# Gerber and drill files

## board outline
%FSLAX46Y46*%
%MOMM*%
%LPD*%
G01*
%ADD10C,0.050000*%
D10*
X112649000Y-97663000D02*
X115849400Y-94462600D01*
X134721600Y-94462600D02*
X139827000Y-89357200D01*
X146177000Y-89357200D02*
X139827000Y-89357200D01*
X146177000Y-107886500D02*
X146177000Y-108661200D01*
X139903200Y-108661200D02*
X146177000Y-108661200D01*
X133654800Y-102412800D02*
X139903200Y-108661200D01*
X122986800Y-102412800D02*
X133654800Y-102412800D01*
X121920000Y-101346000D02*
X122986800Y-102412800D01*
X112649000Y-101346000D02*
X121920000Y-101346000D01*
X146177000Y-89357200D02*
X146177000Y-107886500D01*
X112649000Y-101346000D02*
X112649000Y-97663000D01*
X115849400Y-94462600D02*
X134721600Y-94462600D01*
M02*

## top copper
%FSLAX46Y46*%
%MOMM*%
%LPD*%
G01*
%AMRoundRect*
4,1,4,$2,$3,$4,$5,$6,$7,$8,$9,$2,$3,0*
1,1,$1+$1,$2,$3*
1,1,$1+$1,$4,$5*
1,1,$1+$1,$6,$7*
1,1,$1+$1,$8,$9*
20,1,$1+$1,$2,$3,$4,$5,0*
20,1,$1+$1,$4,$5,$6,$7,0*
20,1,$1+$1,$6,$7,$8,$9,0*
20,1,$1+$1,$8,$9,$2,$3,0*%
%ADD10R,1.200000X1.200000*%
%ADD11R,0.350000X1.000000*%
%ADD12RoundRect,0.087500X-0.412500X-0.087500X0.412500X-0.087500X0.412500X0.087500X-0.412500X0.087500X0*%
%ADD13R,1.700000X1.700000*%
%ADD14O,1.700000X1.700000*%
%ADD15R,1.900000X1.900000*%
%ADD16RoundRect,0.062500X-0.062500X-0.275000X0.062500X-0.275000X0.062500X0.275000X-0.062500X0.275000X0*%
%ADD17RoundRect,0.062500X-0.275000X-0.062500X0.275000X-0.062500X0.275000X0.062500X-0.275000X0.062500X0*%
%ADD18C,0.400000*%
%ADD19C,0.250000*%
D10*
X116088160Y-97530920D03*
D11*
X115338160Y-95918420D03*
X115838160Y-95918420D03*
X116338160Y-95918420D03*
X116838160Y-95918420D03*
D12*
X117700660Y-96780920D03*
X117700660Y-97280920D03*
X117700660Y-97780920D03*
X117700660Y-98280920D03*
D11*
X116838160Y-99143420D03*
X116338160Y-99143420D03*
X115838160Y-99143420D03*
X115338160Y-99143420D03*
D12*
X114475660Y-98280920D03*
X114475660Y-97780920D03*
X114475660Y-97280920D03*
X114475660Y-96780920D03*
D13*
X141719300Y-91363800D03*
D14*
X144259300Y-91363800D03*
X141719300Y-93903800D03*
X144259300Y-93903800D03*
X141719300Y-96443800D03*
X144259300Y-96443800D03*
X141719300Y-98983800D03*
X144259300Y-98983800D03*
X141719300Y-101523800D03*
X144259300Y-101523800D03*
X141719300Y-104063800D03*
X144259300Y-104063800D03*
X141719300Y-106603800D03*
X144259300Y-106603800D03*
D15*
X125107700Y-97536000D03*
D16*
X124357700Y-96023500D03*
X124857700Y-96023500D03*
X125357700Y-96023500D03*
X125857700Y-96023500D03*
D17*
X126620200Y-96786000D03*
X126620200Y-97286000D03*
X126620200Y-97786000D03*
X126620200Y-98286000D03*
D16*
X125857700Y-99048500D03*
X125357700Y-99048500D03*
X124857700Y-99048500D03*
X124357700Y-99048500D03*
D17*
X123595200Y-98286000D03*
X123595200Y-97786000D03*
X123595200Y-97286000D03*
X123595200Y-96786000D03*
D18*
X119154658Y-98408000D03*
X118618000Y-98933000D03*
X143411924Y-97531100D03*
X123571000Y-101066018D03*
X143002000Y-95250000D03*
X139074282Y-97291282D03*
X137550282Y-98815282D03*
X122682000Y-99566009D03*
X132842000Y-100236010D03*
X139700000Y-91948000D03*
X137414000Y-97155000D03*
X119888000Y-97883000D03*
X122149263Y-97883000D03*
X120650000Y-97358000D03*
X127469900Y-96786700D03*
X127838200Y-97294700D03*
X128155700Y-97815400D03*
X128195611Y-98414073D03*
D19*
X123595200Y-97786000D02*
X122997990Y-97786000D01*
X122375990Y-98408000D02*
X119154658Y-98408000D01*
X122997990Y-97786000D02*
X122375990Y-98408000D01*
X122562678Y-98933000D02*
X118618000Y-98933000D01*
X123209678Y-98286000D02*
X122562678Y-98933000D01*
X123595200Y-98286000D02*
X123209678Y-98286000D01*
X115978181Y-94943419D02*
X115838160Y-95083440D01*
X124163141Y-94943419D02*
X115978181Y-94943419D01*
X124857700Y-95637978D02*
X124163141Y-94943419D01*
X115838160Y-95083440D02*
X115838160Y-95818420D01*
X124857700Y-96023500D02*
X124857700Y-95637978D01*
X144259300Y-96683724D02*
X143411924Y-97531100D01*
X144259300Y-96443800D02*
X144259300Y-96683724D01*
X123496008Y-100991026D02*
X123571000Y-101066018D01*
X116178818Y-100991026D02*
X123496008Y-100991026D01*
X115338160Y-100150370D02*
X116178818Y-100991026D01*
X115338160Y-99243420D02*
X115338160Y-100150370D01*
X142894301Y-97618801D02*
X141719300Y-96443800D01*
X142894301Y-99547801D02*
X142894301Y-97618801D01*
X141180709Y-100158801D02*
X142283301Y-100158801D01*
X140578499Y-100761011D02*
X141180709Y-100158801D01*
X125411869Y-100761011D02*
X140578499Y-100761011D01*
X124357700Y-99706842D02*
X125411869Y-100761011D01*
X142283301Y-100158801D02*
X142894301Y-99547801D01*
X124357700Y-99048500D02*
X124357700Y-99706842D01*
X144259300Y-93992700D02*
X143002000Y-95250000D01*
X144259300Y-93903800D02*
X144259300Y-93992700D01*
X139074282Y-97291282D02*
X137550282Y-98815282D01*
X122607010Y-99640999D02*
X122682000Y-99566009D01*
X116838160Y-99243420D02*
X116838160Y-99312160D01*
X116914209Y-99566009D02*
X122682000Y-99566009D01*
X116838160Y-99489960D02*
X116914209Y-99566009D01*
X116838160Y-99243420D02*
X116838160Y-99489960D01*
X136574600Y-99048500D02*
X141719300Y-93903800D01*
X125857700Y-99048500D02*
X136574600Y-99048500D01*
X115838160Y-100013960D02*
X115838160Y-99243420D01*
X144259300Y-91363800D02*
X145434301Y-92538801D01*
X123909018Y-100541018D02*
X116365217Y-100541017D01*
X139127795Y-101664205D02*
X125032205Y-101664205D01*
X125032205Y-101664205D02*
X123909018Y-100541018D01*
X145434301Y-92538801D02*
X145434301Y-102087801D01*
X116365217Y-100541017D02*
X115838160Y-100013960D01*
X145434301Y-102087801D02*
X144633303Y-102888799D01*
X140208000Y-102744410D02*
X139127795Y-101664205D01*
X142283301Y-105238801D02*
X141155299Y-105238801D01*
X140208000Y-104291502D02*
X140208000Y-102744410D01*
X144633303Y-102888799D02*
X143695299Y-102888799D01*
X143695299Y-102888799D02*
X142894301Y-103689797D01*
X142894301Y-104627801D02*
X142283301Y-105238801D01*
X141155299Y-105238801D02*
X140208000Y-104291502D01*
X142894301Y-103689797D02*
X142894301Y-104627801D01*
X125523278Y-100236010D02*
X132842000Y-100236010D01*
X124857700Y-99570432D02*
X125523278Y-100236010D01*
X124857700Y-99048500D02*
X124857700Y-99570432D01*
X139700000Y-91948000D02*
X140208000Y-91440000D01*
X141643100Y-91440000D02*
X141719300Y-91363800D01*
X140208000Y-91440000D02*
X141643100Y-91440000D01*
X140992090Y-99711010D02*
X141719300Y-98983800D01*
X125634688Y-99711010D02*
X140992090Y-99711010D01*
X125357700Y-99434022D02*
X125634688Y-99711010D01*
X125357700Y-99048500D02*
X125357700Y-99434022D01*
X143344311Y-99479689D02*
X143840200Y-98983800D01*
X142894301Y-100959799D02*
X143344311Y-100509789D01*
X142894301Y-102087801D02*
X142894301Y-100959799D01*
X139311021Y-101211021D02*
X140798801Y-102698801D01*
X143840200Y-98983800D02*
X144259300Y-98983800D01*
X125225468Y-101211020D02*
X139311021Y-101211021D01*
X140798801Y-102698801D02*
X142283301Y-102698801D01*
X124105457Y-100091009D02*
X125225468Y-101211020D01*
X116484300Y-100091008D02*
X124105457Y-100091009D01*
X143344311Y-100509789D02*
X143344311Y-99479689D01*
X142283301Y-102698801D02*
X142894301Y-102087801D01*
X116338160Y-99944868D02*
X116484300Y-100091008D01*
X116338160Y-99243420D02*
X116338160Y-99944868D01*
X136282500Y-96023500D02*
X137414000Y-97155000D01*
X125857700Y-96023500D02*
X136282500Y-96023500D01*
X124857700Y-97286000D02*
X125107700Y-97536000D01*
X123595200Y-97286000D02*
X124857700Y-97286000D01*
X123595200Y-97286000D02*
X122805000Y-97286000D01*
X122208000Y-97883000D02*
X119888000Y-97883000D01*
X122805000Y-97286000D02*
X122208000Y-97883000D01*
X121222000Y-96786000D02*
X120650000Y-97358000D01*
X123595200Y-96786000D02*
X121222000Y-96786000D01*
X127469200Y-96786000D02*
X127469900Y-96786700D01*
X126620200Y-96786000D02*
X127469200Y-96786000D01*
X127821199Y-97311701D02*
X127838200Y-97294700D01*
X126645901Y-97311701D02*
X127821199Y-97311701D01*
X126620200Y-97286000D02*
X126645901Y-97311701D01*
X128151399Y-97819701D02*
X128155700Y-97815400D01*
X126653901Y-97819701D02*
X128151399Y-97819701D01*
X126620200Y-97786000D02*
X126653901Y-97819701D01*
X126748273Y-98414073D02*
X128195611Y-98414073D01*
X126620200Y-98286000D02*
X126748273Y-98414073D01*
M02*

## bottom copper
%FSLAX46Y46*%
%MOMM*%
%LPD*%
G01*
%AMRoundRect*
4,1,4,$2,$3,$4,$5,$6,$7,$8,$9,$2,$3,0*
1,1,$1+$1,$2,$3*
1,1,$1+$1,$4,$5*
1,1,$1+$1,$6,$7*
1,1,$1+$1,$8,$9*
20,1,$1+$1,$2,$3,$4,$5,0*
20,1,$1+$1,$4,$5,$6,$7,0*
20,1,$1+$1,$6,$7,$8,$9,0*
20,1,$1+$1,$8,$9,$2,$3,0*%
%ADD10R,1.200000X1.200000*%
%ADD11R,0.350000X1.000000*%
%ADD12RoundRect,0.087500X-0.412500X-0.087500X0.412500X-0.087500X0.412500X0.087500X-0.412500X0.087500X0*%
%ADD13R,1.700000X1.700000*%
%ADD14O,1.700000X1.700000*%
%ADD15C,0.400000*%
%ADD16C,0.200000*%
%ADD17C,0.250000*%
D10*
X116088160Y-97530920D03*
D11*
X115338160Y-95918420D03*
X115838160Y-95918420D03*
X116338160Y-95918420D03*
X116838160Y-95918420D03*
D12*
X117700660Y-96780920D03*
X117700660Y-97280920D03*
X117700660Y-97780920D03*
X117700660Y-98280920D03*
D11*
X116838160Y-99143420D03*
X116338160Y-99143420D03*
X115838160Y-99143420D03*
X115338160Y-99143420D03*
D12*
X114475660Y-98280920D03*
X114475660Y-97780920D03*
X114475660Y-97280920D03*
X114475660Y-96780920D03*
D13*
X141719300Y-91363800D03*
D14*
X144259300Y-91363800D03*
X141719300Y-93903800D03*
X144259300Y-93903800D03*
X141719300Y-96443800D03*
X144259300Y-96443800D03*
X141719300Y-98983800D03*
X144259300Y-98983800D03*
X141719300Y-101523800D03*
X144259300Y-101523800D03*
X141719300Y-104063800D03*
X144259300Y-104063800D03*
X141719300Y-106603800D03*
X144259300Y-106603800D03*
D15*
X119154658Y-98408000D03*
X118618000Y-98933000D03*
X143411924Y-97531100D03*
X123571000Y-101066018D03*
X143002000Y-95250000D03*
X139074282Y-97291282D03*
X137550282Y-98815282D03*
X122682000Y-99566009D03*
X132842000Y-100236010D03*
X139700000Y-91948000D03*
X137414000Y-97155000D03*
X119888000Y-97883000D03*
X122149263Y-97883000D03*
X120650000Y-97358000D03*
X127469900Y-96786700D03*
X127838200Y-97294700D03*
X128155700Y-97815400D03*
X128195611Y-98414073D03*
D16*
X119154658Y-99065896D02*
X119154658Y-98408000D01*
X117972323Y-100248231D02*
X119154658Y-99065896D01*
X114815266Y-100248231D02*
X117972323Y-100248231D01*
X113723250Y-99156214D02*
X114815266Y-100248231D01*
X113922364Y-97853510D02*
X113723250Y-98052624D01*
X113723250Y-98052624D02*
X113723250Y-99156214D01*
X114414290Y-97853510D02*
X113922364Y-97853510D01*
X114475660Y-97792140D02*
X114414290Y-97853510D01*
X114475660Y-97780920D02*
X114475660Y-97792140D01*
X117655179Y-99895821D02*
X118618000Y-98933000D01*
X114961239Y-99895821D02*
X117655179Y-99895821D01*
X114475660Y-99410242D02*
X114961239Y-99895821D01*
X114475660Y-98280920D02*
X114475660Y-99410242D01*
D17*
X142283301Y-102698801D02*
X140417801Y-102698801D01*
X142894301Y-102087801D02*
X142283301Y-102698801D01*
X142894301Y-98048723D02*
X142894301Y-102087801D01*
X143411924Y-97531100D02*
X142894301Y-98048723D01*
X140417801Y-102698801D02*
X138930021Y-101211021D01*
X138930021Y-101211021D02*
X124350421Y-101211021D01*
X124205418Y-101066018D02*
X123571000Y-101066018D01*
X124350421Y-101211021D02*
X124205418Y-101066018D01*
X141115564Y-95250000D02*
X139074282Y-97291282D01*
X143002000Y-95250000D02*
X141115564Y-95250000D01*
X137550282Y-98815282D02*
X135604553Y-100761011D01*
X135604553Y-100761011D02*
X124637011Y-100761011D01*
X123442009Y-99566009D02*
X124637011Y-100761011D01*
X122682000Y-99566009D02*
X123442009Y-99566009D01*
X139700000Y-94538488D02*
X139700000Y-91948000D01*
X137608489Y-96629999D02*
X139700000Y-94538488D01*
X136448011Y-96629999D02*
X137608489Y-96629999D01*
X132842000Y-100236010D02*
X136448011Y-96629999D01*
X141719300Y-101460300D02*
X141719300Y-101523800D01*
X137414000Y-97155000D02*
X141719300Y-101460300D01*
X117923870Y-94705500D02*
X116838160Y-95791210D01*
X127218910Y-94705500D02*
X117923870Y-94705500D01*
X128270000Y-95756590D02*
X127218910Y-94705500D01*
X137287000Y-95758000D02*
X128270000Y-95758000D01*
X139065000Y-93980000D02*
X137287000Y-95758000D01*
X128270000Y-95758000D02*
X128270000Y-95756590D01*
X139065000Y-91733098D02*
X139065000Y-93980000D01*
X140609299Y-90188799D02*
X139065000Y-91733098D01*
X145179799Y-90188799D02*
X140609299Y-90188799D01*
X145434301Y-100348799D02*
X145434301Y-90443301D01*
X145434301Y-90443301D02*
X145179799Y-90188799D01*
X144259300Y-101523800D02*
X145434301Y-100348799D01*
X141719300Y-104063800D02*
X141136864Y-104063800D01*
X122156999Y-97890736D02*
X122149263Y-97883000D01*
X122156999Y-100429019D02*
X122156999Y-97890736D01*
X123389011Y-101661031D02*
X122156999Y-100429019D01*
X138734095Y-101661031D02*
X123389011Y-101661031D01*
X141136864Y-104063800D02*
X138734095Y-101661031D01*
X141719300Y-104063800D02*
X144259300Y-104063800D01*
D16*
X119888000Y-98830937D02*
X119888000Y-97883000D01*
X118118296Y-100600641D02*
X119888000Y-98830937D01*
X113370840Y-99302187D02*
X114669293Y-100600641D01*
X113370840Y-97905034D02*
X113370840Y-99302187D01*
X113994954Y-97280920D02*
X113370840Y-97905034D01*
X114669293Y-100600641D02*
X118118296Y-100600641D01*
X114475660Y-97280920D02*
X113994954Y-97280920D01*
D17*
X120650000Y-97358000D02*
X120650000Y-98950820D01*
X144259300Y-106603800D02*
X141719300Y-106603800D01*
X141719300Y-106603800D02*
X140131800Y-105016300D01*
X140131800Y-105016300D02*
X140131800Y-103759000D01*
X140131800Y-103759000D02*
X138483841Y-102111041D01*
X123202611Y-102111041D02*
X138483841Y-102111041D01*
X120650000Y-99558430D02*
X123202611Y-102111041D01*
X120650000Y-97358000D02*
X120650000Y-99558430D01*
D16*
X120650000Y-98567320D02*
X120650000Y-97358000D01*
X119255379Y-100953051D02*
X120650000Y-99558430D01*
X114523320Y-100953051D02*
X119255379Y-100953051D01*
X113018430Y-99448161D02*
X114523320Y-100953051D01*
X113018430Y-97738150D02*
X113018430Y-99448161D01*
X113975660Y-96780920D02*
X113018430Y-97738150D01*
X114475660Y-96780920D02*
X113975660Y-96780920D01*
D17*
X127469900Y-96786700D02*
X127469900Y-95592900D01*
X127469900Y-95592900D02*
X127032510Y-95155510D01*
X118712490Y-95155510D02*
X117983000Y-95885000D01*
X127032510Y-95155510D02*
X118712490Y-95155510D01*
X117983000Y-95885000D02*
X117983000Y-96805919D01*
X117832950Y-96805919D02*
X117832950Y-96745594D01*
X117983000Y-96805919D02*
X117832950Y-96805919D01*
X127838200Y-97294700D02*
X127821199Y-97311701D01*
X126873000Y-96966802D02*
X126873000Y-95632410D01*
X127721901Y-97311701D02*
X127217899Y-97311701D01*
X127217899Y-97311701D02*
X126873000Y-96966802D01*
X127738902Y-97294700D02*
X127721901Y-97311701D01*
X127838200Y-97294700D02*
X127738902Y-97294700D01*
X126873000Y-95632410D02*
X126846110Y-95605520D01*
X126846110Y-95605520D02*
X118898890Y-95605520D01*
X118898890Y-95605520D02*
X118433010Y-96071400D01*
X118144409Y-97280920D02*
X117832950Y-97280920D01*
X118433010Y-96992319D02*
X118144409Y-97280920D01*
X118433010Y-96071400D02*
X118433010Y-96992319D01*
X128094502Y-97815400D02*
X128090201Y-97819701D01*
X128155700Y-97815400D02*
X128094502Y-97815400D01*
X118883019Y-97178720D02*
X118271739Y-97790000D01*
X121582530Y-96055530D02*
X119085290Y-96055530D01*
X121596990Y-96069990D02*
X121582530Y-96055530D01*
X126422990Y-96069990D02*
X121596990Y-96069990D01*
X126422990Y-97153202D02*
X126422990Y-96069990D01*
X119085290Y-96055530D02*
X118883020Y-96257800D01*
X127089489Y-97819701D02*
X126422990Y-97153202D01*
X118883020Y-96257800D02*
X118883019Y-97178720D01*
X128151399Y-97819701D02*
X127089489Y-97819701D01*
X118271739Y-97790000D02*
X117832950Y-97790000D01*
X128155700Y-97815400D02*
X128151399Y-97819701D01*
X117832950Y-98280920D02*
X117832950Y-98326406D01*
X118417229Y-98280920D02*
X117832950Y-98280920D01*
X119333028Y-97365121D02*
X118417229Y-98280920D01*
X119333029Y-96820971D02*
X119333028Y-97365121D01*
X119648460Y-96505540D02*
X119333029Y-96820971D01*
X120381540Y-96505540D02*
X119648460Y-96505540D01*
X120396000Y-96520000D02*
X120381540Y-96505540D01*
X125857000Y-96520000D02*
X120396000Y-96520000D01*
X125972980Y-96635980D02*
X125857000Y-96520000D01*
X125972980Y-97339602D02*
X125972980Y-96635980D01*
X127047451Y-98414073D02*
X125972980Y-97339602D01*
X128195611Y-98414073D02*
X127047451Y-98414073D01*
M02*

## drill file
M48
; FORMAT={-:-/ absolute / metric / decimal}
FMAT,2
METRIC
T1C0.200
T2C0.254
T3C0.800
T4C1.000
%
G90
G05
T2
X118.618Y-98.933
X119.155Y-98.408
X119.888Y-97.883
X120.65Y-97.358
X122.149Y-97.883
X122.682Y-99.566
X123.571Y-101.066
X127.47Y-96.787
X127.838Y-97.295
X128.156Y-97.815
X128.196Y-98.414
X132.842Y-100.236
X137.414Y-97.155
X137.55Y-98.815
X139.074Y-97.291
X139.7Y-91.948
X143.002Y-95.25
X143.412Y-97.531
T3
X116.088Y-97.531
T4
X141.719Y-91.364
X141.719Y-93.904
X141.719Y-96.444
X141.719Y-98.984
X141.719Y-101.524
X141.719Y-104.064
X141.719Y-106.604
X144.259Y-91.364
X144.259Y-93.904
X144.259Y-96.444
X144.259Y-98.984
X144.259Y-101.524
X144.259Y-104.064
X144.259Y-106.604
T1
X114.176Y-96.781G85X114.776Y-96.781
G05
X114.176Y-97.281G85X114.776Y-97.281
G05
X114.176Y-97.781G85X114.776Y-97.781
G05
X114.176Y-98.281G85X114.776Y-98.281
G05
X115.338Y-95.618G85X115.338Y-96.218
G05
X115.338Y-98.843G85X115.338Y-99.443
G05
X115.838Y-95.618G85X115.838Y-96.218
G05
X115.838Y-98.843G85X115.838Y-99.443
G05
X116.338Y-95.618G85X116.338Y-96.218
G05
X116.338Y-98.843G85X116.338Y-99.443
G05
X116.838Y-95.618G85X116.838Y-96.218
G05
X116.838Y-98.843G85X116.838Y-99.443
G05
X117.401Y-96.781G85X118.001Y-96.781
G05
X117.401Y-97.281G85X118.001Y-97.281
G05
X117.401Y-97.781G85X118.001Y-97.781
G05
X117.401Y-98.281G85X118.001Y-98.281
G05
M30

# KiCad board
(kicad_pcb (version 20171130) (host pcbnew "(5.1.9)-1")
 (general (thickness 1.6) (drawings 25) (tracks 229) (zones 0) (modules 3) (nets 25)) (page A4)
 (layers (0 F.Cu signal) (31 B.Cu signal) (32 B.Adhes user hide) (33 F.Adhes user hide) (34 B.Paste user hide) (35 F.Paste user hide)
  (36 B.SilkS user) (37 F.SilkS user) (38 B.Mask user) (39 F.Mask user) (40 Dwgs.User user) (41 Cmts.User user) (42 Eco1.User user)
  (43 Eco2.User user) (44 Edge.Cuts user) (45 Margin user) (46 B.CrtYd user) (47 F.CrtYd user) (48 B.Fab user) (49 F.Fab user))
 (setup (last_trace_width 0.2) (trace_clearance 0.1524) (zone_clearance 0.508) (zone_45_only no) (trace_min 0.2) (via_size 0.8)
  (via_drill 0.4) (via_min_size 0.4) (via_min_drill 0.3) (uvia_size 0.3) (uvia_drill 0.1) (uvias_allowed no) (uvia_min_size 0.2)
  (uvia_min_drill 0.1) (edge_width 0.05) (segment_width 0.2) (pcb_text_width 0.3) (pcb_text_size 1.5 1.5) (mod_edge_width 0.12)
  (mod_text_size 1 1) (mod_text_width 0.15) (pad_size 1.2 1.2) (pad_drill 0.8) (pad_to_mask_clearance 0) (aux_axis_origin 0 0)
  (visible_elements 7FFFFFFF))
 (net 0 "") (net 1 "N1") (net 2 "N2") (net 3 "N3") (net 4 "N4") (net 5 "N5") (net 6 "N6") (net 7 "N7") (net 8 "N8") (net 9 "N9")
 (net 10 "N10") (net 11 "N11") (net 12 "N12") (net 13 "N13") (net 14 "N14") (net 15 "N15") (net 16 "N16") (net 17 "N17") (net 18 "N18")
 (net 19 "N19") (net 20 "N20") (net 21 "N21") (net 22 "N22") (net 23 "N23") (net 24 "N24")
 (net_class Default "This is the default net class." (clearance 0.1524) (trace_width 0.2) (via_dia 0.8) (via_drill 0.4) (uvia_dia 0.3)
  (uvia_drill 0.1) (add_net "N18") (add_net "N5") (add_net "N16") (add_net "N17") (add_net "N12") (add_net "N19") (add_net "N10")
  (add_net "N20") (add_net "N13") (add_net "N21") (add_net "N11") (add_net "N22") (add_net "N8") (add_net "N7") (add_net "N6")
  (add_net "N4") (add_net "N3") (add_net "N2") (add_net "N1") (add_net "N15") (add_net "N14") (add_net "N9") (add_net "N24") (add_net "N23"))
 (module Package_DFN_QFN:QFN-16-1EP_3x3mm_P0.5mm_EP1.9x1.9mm (layer F.Cu) (at 116.08816 97.53092)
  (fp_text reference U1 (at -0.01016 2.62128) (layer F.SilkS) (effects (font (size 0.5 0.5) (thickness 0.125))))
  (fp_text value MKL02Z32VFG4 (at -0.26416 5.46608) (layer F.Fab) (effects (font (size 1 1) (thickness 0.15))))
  (pad "" smd roundrect (at 0.475 0.475) (size 0.77 0.77) (layers F.Paste) (roundrect_rratio 0.25))
  (pad "" smd roundrect (at 0.475 -0.475) (size 0.77 0.77) (layers F.Paste) (roundrect_rratio 0.25))
  (pad "" smd roundrect (at -0.475 0.475) (size 0.77 0.77) (layers F.Paste) (roundrect_rratio 0.25))
  (pad "" smd roundrect (at -0.475 -0.475) (size 0.77 0.77) (layers F.Paste) (roundrect_rratio 0.25))
  (pad 17 thru_hole rect (at 0 0) (size 1.2 1.2) (drill 0.8) (layers *.Cu *.Mask) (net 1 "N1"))
  (pad 16 thru_hole rect (at -0.75 -1.6125) (size 0.35 1) (drill oval 0.2 0.8) (layers *.Cu *.Mask) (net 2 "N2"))
  (pad 15 thru_hole rect (at -0.25 -1.6125) (size 0.35 1) (drill oval 0.2 0.8) (layers *.Cu *.Mask) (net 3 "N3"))
  (pad 14 thru_hole rect (at 0.25 -1.6125) (size 0.35 1) (drill oval 0.2 0.8) (layers *.Cu *.Mask) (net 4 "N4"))
  (pad 13 thru_hole rect (at 0.75 -1.6125) (size 0.35 1) (drill oval 0.2 0.8) (layers *.Cu *.Mask) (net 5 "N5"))
  (pad 12 thru_hole roundrect (at 1.6125 -0.75) (size 1 0.35) (drill oval 0.8 0.2) (layers *.Cu *.Mask) (roundrect_rratio 0.25) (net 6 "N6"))
  (pad 11 thru_hole roundrect (at 1.6125 -0.25) (size 1 0.35) (drill oval 0.8 0.2) (layers *.Cu *.Mask) (roundrect_rratio 0.25) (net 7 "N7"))
  (pad 10 thru_hole roundrect (at 1.6125 0.25) (size 1 0.35) (drill oval 0.8 0.2) (layers *.Cu *.Mask) (roundrect_rratio 0.25) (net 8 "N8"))
  (pad 9 thru_hole roundrect (at 1.6125 0.75) (size 1 0.35) (drill oval 0.8 0.2) (layers *.Cu *.Mask) (roundrect_rratio 0.25) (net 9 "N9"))
  (pad 8 thru_hole rect (at 0.75 1.6125) (size 0.35 1) (drill oval 0.2 0.8) (layers *.Cu *.Mask) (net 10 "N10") (clearance 0.00001))
  (pad 7 thru_hole rect (at 0.25 1.6125) (size 0.35 1) (drill oval 0.2 0.8) (layers *.Cu *.Mask) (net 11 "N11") (clearance 0.000001))
  (pad 6 thru_hole rect (at -0.25 1.6125) (size 0.35 1) (drill oval 0.2 0.8) (layers *.Cu *.Mask) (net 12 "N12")
   (solder_mask_margin 0.000001) (clearance 0.00001))
  (pad 5 thru_hole rect (at -0.75 1.6125) (size 0.35 1) (drill oval 0.2 0.8) (layers *.Cu *.Mask) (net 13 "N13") (clearance 0.00001))
  (pad 4 thru_hole roundrect (at -1.6125 0.75) (size 1 0.35) (drill oval 0.8 0.2) (layers *.Cu *.Mask) (roundrect_rratio 0.25)
   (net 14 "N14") (clearance 0.0001))
  (pad 3 thru_hole roundrect (at -1.6125 0.25) (size 1 0.35) (drill oval 0.8 0.2) (layers *.Cu *.Mask) (roundrect_rratio 0.25)
   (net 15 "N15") (clearance 0.0001))
  (pad 2 thru_hole roundrect (at -1.6125 -0.25) (size 1 0.35) (drill oval 0.8 0.2) (layers *.Cu *.Mask) (roundrect_rratio 0.25)
   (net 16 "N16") (clearance 0.0001))
  (pad 1 thru_hole roundrect (at -1.6125 -0.75) (size 1 0.35) (drill oval 0.8 0.2) (layers *.Cu *.Mask) (roundrect_rratio 0.25)
   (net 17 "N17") (clearance 0.00001)))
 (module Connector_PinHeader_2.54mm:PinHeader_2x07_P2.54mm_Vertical (layer F.Cu) (at 141.7193 91.3638)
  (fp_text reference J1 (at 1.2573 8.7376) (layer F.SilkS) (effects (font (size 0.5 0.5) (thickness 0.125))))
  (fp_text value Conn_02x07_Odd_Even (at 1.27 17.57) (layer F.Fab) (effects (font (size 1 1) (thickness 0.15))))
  (pad 1 thru_hole rect (at 0 0) (size 1.7 1.7) (drill 1) (layers *.Cu *.Mask) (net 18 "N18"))
  (pad 2 thru_hole oval (at 2.54 0) (size 1.7 1.7) (drill 1) (layers *.Cu *.Mask) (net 12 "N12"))
  (pad 3 thru_hole oval (at 0 2.54) (size 1.7 1.7) (drill 1) (layers *.Cu *.Mask) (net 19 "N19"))
  (pad 4 thru_hole oval (at 2.54 2.54) (size 1.7 1.7) (drill 1) (layers *.Cu *.Mask) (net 10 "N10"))
  (pad 5 thru_hole oval (at 0 5.08) (size 1.7 1.7) (drill 1) (layers *.Cu *.Mask) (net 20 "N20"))
  (pad 6 thru_hole oval (at 2.54 5.08) (size 1.7 1.7) (drill 1) (layers *.Cu *.Mask) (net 13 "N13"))
  (pad 7 thru_hole oval (at 0 7.62) (size 1.7 1.7) (drill 1) (layers *.Cu *.Mask) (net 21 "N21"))
  (pad 8 thru_hole oval (at 2.54 7.62) (size 1.7 1.7) (drill 1) (layers *.Cu *.Mask) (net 11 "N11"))
  (pad 9 thru_hole oval (at 0 10.16) (size 1.7 1.7) (drill 1) (layers *.Cu *.Mask) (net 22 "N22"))
  (pad 10 thru_hole oval (at 2.54 10.16) (size 1.7 1.7) (drill 1) (layers *.Cu *.Mask) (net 5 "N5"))
  (pad 11 thru_hole oval (at 0 12.7) (size 1.7 1.7) (drill 1) (layers *.Cu *.Mask) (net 16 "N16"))
  (pad 12 thru_hole oval (at 2.54 12.7) (size 1.7 1.7) (drill 1) (layers *.Cu *.Mask) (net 16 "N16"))
  (pad 13 thru_hole oval (at 0 15.24) (size 1.7 1.7) (drill 1) (layers *.Cu *.Mask) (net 17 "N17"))
  (pad 14 thru_hole oval (at 2.54 15.24) (size 1.7 1.7) (drill 1) (layers *.Cu *.Mask) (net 17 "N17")))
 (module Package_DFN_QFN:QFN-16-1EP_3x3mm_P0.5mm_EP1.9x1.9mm (layer F.Cu) (at 125.1077 97.536)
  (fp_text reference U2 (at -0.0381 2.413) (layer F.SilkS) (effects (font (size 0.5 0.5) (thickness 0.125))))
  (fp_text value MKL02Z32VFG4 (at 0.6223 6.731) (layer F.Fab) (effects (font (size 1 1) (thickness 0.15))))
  (pad "" smd roundrect (at 0.475 0.475) (size 0.77 0.77) (layers F.Paste) (roundrect_rratio 0.25))
  (pad "" smd roundrect (at 0.475 -0.475) (size 0.77 0.77) (layers F.Paste) (roundrect_rratio 0.25))
  (pad "" smd roundrect (at -0.475 0.475) (size 0.77 0.77) (layers F.Paste) (roundrect_rratio 0.25))
  (pad "" smd roundrect (at -0.475 -0.475) (size 0.77 0.77) (layers F.Paste) (roundrect_rratio 0.25))
  (pad 17 smd rect (at 0 0) (size 1.9 1.9) (layers F.Cu F.Mask) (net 16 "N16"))
  (pad 16 smd roundrect (at -0.75 -1.5125) (size 0.25 0.675) (layers F.Cu F.Paste F.Mask) (roundrect_rratio 0.25) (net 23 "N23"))
  (pad 15 smd roundrect (at -0.25 -1.5125) (size 0.25 0.675) (layers F.Cu F.Paste F.Mask) (roundrect_rratio 0.25) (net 3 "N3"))
  (pad 14 smd roundrect (at 0.25 -1.5125) (size 0.25 0.675) (layers F.Cu F.Paste F.Mask) (roundrect_rratio 0.25) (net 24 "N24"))
  (pad 13 smd roundrect (at 0.75 -1.5125) (size 0.25 0.675) (layers F.Cu F.Paste F.Mask) (roundrect_rratio 0.25) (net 22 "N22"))
  (pad 12 smd roundrect (at 1.5125 -0.75) (size 0.675 0.25) (layers F.Cu F.Paste F.Mask) (roundrect_rratio 0.25) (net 6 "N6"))
  (pad 11 smd roundrect (at 1.5125 -0.25) (size 0.675 0.25) (layers F.Cu F.Paste F.Mask) (roundrect_rratio 0.25) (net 7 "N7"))
  (pad 10 smd roundrect (at 1.5125 0.25) (size 0.675 0.25) (layers F.Cu F.Paste F.Mask) (roundrect_rratio 0.25) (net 8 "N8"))
  (pad 9 smd roundrect (at 1.5125 0.75) (size 0.675 0.25) (layers F.Cu F.Paste F.Mask) (roundrect_rratio 0.25) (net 9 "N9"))
  (pad 8 smd roundrect (at 0.75 1.5125) (size 0.25 0.675) (layers F.Cu F.Paste F.Mask) (roundrect_rratio 0.25) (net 19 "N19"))
  (pad 7 smd roundrect (at 0.25 1.5125) (size 0.25 0.675) (layers F.Cu F.Paste F.Mask) (roundrect_rratio 0.25) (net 21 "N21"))
  (pad 6 smd roundrect (at -0.25 1.5125) (size 0.25 0.675) (layers F.Cu F.Paste F.Mask) (roundrect_rratio 0.25) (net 18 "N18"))
  (pad 5 smd roundrect (at -0.75 1.5125) (size 0.25 0.675) (layers F.Cu F.Paste F.Mask) (roundrect_rratio 0.25) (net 20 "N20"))
  (pad 4 smd roundrect (at -1.5125 0.75) (size 0.675 0.25) (layers F.Cu F.Paste F.Mask) (roundrect_rratio 0.25) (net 14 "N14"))
  (pad 3 smd roundrect (at -1.5125 0.25) (size 0.675 0.25) (layers F.Cu F.Paste F.Mask) (roundrect_rratio 0.25) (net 15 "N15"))
  (pad 2 smd roundrect (at -1.5125 -0.25) (size 0.675 0.25) (layers F.Cu F.Paste F.Mask) (roundrect_rratio 0.25) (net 16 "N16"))
  (pad 1 smd roundrect (at -1.5125 -0.75) (size 0.675 0.25) (layers F.Cu F.Paste F.Mask) (roundrect_rratio 0.25) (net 17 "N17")))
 (gr_line (start 112.649 97.663) (end 115.8494 94.4626) (layer Edge.Cuts) (width 0.05))
 (gr_line (start 134.7216 94.4626) (end 139.827 89.3572) (layer Edge.Cuts) (width 0.05))
 (gr_line (start 146.177 89.3572) (end 139.827 89.3572) (layer Edge.Cuts) (width 0.05))
 (gr_line (start 146.177 107.8865) (end 146.177 108.6612) (layer Edge.Cuts) (width 0.05))
 (gr_line (start 139.9032 108.6612) (end 146.177 108.6612) (layer Edge.Cuts) (width 0.05))
 (gr_line (start 133.6548 102.4128) (end 139.9032 108.6612) (layer Edge.Cuts) (width 0.05))
 (gr_line (start 122.9868 102.4128) (end 133.6548 102.4128) (layer Edge.Cuts) (width 0.05))
 (gr_line (start 121.92 101.346) (end 122.9868 102.4128) (layer Edge.Cuts) (width 0.05))
 (gr_line (start 112.649 101.346) (end 121.92 101.346) (layer Edge.Cuts) (width 0.05))
 (gr_line (start 146.177 89.3572) (end 146.177 107.8865) (layer Edge.Cuts) (width 0.05))
 (gr_line (start 112.649 101.346) (end 112.649 97.663) (layer Edge.Cuts) (width 0.05))
 (gr_line (start 115.8494 94.4626) (end 134.7216 94.4626) (layer Edge.Cuts) (width 0.05))
 (segment (start 123.5952 97.786) (end 122.99799 97.786) (width 0.25) (layer F.Cu) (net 15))
 (via (at 119.154658 98.408) (size 0.4) (drill 0.254) (layers F.Cu B.Cu) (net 15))
 (segment (start 122.37599 98.408) (end 119.154658 98.408) (width 0.25) (layer F.Cu) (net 15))
 (segment (start 122.99799 97.786) (end 122.37599 98.408) (width 0.25) (layer F.Cu) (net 15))
 (segment (start 119.154658 99.065896) (end 119.154658 98.408) (width 0.2) (layer B.Cu) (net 15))
 (segment (start 117.972323 100.248231) (end 119.154658 99.065896) (width 0.2) (layer B.Cu) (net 15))
 (segment (start 114.815266 100.248231) (end 117.972323 100.248231) (width 0.2) (layer B.Cu) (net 15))
 (segment (start 113.72325 99.156214) (end 114.815266 100.248231) (width 0.2) (layer B.Cu) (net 15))
 (segment (start 113.922364 97.85351) (end 113.72325 98.052624) (width 0.2) (layer B.Cu) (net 15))
 (segment (start 113.72325 98.052624) (end 113.72325 99.156214) (width 0.2) (layer B.Cu) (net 15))
 (segment (start 114.41429 97.85351) (end 113.922364 97.85351) (width 0.2) (layer B.Cu) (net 15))
 (segment (start 114.47566 97.79214) (end 114.41429 97.85351) (width 0.2) (layer B.Cu) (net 15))
 (segment (start 114.47566 97.78092) (end 114.47566 97.79214) (width 0.2) (layer B.Cu) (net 15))
 (via (at 118.618 98.933) (size 0.4) (drill 0.254) (layers F.Cu B.Cu) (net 14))
 (segment (start 122.562678 98.933) (end 118.618 98.933) (width 0.25) (layer F.Cu) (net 14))
 (segment (start 123.209678 98.286) (end 122.562678 98.933) (width 0.25) (layer F.Cu) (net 14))
 (segment (start 123.5952 98.286) (end 123.209678 98.286) (width 0.25) (layer F.Cu) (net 14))
 (segment (start 117.655179 99.895821) (end 118.618 98.933) (width 0.2) (layer B.Cu) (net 14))
 (segment (start 114.961239 99.895821) (end 117.655179 99.895821) (width 0.2) (layer B.Cu) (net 14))
 (segment (start 114.47566 99.410242) (end 114.961239 99.895821) (width 0.2) (layer B.Cu) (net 14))
 (segment (start 114.47566 98.28092) (end 114.47566 99.410242) (width 0.2) (layer B.Cu) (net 14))
 (segment (start 115.978181 94.943419) (end 115.83816 95.08344) (width 0.25) (layer F.Cu) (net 3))
 (segment (start 124.163141 94.943419) (end 115.978181 94.943419) (width 0.25) (layer F.Cu) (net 3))
 (segment (start 124.8577 95.637978) (end 124.163141 94.943419) (width 0.25) (layer F.Cu) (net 3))
 (segment (start 115.83816 95.08344) (end 115.83816 95.81842) (width 0.25) (layer F.Cu) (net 3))
 (segment (start 124.8577 96.0235) (end 124.8577 95.637978) (width 0.25) (layer F.Cu) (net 3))
 (via (at 143.411924 97.5311) (size 0.4) (drill 0.254) (layers F.Cu B.Cu) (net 13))
 (segment (start 144.2593 96.683724) (end 143.411924 97.5311) (width 0.25) (layer F.Cu) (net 13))
 (segment (start 144.2593 96.4438) (end 144.2593 96.683724) (width 0.25) (layer F.Cu) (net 13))
 (segment (start 142.283301 102.698801) (end 140.417801 102.698801) (width 0.25) (layer B.Cu) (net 13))
 (segment (start 142.894301 102.087801) (end 142.283301 102.698801) (width 0.25) (layer B.Cu) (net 13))
 (segment (start 142.894301 98.048723) (end 142.894301 102.087801) (width 0.25) (layer B.Cu) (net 13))
 (segment (start 143.411924 97.5311) (end 142.894301 98.048723) (width 0.25) (layer B.Cu) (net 13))
 (segment (start 140.417801 102.698801) (end 138.930021 101.211021) (width 0.25) (layer B.Cu) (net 13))
 (via (at 123.571 101.066018) (size 0.4) (drill 0.254) (layers F.Cu B.Cu) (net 13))
 (segment (start 138.930021 101.211021) (end 124.350421 101.211021) (width 0.25) (layer B.Cu) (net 13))
 (segment (start 124.205418 101.066018) (end 123.571 101.066018) (width 0.25) (layer B.Cu) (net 13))
 (segment (start 124.350421 101.211021) (end 124.205418 101.066018) (width 0.25) (layer B.Cu) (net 13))
 (segment (start 123.496008 100.991026) (end 123.571 101.066018) (width 0.25) (layer F.Cu) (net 13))
 (segment (start 116.178818 100.991026) (end 123.496008 100.991026) (width 0.25) (layer F.Cu) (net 13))
 (segment (start 115.33816 100.15037) (end 116.178818 100.991026) (width 0.25) (layer F.Cu) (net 13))
 (segment (start 115.33816 99.24342) (end 115.33816 100.15037) (width 0.25) (layer F.Cu) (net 13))
 (segment (start 142.894301 97.618801) (end 141.7193 96.4438) (width 0.25) (layer F.Cu) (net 20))
 (segment (start 142.894301 99.547801) (end 142.894301 97.618801) (width 0.25) (layer F.Cu) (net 20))
 (segment (start 141.180709 100.158801) (end 142.283301 100.158801) (width 0.25) (layer F.Cu) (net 20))
 (segment (start 140.578499 100.761011) (end 141.180709 100.158801) (width 0.25) (layer F.Cu) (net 20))
 (segment (start 125.411869 100.761011) (end 140.578499 100.761011) (width 0.25) (layer F.Cu) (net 20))
 (segment (start 124.3577 99.706842) (end 125.411869 100.761011) (width 0.25) (layer F.Cu) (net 20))
 (segment (start 142.283301 100.158801) (end 142.894301 99.547801) (width 0.25) (layer F.Cu) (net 20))
 (segment (start 124.3577 99.0485) (end 124.3577 99.706842) (width 0.25) (layer F.Cu) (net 20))
 (via (at 143.002 95.25) (size 0.4) (drill 0.254) (layers F.Cu B.Cu) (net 10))
 (segment (start 144.2593 93.9927) (end 143.002 95.25) (width 0.25) (layer F.Cu) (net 10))
 (segment (start 144.2593 93.9038) (end 144.2593 93.9927) (width 0.25) (layer F.Cu) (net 10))
 (via (at 139.074282 97.291282) (size 0.4) (drill 0.254) (layers F.Cu B.Cu) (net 10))
 (segment (start 141.115564 95.25) (end 139.074282 97.291282) (width 0.25) (layer B.Cu) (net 10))
 (segment (start 143.002 95.25) (end 141.115564 95.25) (width 0.25) (layer B.Cu) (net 10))
 (via (at 137.550282 98.815282) (size 0.4) (drill 0.254) (layers F.Cu B.Cu) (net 10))
 (segment (start 139.074282 97.291282) (end 137.550282 98.815282) (width 0.25) (layer F.Cu) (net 10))
 (segment (start 137.550282 98.815282) (end 135.604553 100.761011) (width 0.25) (layer B.Cu) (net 10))
 (segment (start 135.604553 100.761011) (end 124.637011 100.761011) (width 0.25) (layer B.Cu) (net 10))
 (via (at 122.682 99.566009) (size 0.4) (drill 0.254) (layers F.Cu B.Cu) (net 10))
 (segment (start 123.442009 99.566009) (end 124.637011 100.761011) (width 0.25) (layer B.Cu) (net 10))
 (segment (start 122.682 99.566009) (end 123.442009 99.566009) (width 0.25) (layer B.Cu) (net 10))
 (segment (start 122.60701 99.640999) (end 122.682 99.566009) (width 0.25) (layer F.Cu) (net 10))
 (segment (start 116.83816 99.24342) (end 116.83816 99.31216) (width 0.25) (layer F.Cu) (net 10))
 (segment (start 116.914209 99.566009) (end 122.682 99.566009) (width 0.25) (layer F.Cu) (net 10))
 (segment (start 116.83816 99.48996) (end 116.914209 99.566009) (width 0.25) (layer F.Cu) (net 10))
 (segment (start 116.83816 99.24342) (end 116.83816 99.48996) (width 0.25) (layer F.Cu) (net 10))
 (segment (start 136.5746 99.0485) (end 141.7193 93.9038) (width 0.25) (layer F.Cu) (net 19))
 (segment (start 125.8577 99.0485) (end 136.5746 99.0485) (width 0.25) (layer F.Cu) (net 19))
 (segment (start 115.83816 100.01396) (end 115.83816 99.24342) (width 0.25) (layer F.Cu) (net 12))
 (segment (start 144.2593 91.3638) (end 145.434301 92.538801) (width 0.25) (layer F.Cu) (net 12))
 (segment (start 123.909018 100.541018) (end 116.365217 100.541017) (width 0.25) (layer F.Cu) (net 12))
 (segment (start 139.127795 101.664205) (end 125.032205 101.664205) (width 0.25) (layer F.Cu) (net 12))
 (segment (start 125.032205 101.664205) (end 123.909018 100.541018) (width 0.25) (layer F.Cu) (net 12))
 (segment (start 145.434301 92.538801) (end 145.434301 102.087801) (width 0.25) (layer F.Cu) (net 12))
 (segment (start 116.365217 100.541017) (end 115.83816 100.01396) (width 0.25) (layer F.Cu) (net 12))
 (segment (start 145.434301 102.087801) (end 144.633303 102.888799) (width 0.25) (layer F.Cu) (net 12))
 (segment (start 140.208 102.74441) (end 139.127795 101.664205) (width 0.25) (layer F.Cu) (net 12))
 (segment (start 142.283301 105.238801) (end 141.155299 105.238801) (width 0.25) (layer F.Cu) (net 12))
 (segment (start 140.208 104.291502) (end 140.208 102.74441) (width 0.25) (layer F.Cu) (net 12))
 (segment (start 144.633303 102.888799) (end 143.695299 102.888799) (width 0.25) (layer F.Cu) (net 12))
 (segment (start 143.695299 102.888799) (end 142.894301 103.689797) (width 0.25) (layer F.Cu) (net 12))
 (segment (start 142.894301 104.627801) (end 142.283301 105.238801) (width 0.25) (layer F.Cu) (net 12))
 (segment (start 141.155299 105.238801) (end 140.208 104.291502) (width 0.25) (layer F.Cu) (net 12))
 (segment (start 142.894301 103.689797) (end 142.894301 104.627801) (width 0.25) (layer F.Cu) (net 12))
 (via (at 132.842 100.23601) (size 0.4) (drill 0.254) (layers F.Cu B.Cu) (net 18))
 (segment (start 125.523278 100.23601) (end 132.842 100.23601) (width 0.25) (layer F.Cu) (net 18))
 (segment (start 124.8577 99.570432) (end 125.523278 100.23601) (width 0.25) (layer F.Cu) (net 18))
 (segment (start 124.8577 99.0485) (end 124.8577 99.570432) (width 0.25) (layer F.Cu) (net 18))
 (via (at 139.7 91.948) (size 0.4) (drill 0.254) (layers F.Cu B.Cu) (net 18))
 (segment (start 139.7 94.538488) (end 139.7 91.948) (width 0.25) (layer B.Cu) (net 18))
 (segment (start 137.608489 96.629999) (end 139.7 94.538488) (width 0.25) (layer B.Cu) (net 18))
 (segment (start 136.448011 96.629999) (end 137.608489 96.629999) (width 0.25) (layer B.Cu) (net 18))
 (segment (start 132.842 100.23601) (end 136.448011 96.629999) (width 0.25) (layer B.Cu) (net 18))
 (segment (start 139.7 91.948) (end 140.208 91.44) (width 0.25) (layer F.Cu) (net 18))
 (segment (start 141.6431 91.44) (end 141.7193 91.3638) (width 0.25) (layer F.Cu) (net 18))
 (segment (start 140.208 91.44) (end 141.6431 91.44) (width 0.25) (layer F.Cu) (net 18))
 (segment (start 140.99209 99.71101) (end 141.7193 98.9838) (width 0.25) (layer F.Cu) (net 21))
 (segment (start 125.634688 99.71101) (end 140.99209 99.71101) (width 0.25) (layer F.Cu) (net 21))
 (segment (start 125.3577 99.434022) (end 125.634688 99.71101) (width 0.25) (layer F.Cu) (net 21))
 (segment (start 125.3577 99.0485) (end 125.3577 99.434022) (width 0.25) (layer F.Cu) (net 21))
 (segment (start 143.344311 99.479689) (end 143.8402 98.9838) (width 0.25) (layer F.Cu) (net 11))
 (segment (start 142.894301 100.959799) (end 143.344311 100.509789) (width 0.25) (layer F.Cu) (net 11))
 (segment (start 142.894301 102.087801) (end 142.894301 100.959799) (width 0.25) (layer F.Cu) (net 11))
 (segment (start 139.311021 101.211021) (end 140.798801 102.698801) (width 0.25) (layer F.Cu) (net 11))
 (segment (start 143.8402 98.9838) (end 144.2593 98.9838) (width 0.25) (layer F.Cu) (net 11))
 (segment (start 125.225468 101.21102) (end 139.311021 101.211021) (width 0.25) (layer F.Cu) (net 11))
 (segment (start 140.798801 102.698801) (end 142.283301 102.698801) (width 0.25) (layer F.Cu) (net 11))
 (segment (start 124.105457 100.091009) (end 125.225468 101.21102) (width 0.25) (layer F.Cu) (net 11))
 (segment (start 116.4843 100.091008) (end 124.105457 100.091009) (width 0.25) (layer F.Cu) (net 11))
 (segment (start 143.344311 100.509789) (end 143.344311 99.479689) (width 0.25) (layer F.Cu) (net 11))
 (segment (start 142.283301 102.698801) (end 142.894301 102.087801) (width 0.25) (layer F.Cu) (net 11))
 (segment (start 116.33816 99.944868) (end 116.4843 100.091008) (width 0.25) (layer F.Cu) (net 11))
 (segment (start 116.33816 99.24342) (end 116.33816 99.944868) (width 0.25) (layer F.Cu) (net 11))
 (via (at 137.414 97.155) (size 0.4) (drill 0.254) (layers F.Cu B.Cu) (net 22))
 (segment (start 136.2825 96.0235) (end 137.414 97.155) (width 0.25) (layer F.Cu) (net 22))
 (segment (start 125.8577 96.0235) (end 136.2825 96.0235) (width 0.25) (layer F.Cu) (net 22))
 (segment (start 141.7193 101.4603) (end 141.7193 101.5238) (width 0.25) (layer B.Cu) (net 22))
 (segment (start 137.414 97.155) (end 141.7193 101.4603) (width 0.25) (layer B.Cu) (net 22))
 (segment (start 117.92387 94.7055) (end 116.83816 95.79121) (width 0.25) (layer B.Cu) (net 5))
 (segment (start 127.21891 94.7055) (end 117.92387 94.7055) (width 0.25) (layer B.Cu) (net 5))
 (segment (start 128.27 95.75659) (end 127.21891 94.7055) (width 0.25) (layer B.Cu) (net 5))
 (segment (start 137.287 95.758) (end 128.27 95.758) (width 0.25) (layer B.Cu) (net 5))
 (segment (start 139.065 93.98) (end 137.287 95.758) (width 0.25) (layer B.Cu) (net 5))
 (segment (start 128.27 95.758) (end 128.27 95.75659) (width 0.25) (layer B.Cu) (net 5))
 (segment (start 139.065 91.733098) (end 139.065 93.98) (width 0.25) (layer B.Cu) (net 5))
 (segment (start 140.609299 90.188799) (end 139.065 91.733098) (width 0.25) (layer B.Cu) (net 5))
 (segment (start 145.179799 90.188799) (end 140.609299 90.188799) (width 0.25) (layer B.Cu) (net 5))
 (segment (start 145.434301 100.348799) (end 145.434301 90.443301) (width 0.25) (layer B.Cu) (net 5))
 (segment (start 145.434301 90.443301) (end 145.179799 90.188799) (width 0.25) (layer B.Cu) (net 5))
 (segment (start 144.2593 101.5238) (end 145.434301 100.348799) (width 0.25) (layer B.Cu) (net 5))
 (segment (start 124.8577 97.286) (end 125.1077 97.536) (width 0.25) (layer F.Cu) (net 16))
 (segment (start 123.5952 97.286) (end 124.8577 97.286) (width 0.25) (layer F.Cu) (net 16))
 (segment (start 123.5952 97.286) (end 122.805 97.286) (width 0.25) (layer F.Cu) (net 16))
 (segment (start 122.208 97.883) (end 119.888 97.883) (width 0.25) (layer F.Cu) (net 16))
 (via (at 119.888 97.883) (size 0.4) (drill 0.254) (layers F.Cu B.Cu) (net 16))
 (segment (start 122.805 97.286) (end 122.208 97.883) (width 0.25) (layer F.Cu) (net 16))
 (segment (start 141.7193 104.0638) (end 141.136864 104.0638) (width 0.25) (layer B.Cu) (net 16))
 (segment (start 122.156999 97.890736) (end 122.149263 97.883) (width 0.25) (layer B.Cu) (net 16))
 (segment (start 122.156999 100.429019) (end 122.156999 97.890736) (width 0.25) (layer B.Cu) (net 16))
 (via (at 122.149263 97.883) (size 0.4) (drill 0.254) (layers F.Cu B.Cu) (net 16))
 (segment (start 123.389011 101.661031) (end 122.156999 100.429019) (width 0.25) (layer B.Cu) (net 16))
 (segment (start 138.734095 101.661031) (end 123.389011 101.661031) (width 0.25) (layer B.Cu) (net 16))
 (segment (start 141.136864 104.0638) (end 138.734095 101.661031) (width 0.25) (layer B.Cu) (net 16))
 (segment (start 141.7193 104.0638) (end 144.2593 104.0638) (width 0.25) (layer B.Cu) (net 16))
 (segment (start 119.888 98.830937) (end 119.888 97.883) (width 0.2) (layer B.Cu) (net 16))
 (segment (start 118.118296 100.600641) (end 119.888 98.830937) (width 0.2) (layer B.Cu) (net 16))
 (segment (start 113.37084 99.302187) (end 114.669293 100.600641) (width 0.2) (layer B.Cu) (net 16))
 (segment (start 113.37084 97.905034) (end 113.37084 99.302187) (width 0.2) (layer B.Cu) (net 16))
 (segment (start 113.994954 97.28092) (end 113.37084 97.905034) (width 0.2) (layer B.Cu) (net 16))
 (segment (start 114.669293 100.600641) (end 118.118296 100.600641) (width 0.2) (layer B.Cu) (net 16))
 (segment (start 114.47566 97.28092) (end 113.994954 97.28092) (width 0.2) (layer B.Cu) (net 16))
 (via (at 120.65 97.358) (size 0.4) (drill 0.254) (layers F.Cu B.Cu) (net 17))
 (segment (start 121.222 96.786) (end 120.65 97.358) (width 0.25) (layer F.Cu) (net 17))
 (segment (start 123.5952 96.786) (end 121.222 96.786) (width 0.25) (layer F.Cu) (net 17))
 (segment (start 120.65 97.358) (end 120.65 98.95082) (width 0.25) (layer B.Cu) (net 17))
 (segment (start 144.2593 106.6038) (end 141.7193 106.6038) (width 0.25) (layer B.Cu) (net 17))
 (segment (start 141.7193 106.6038) (end 140.1318 105.0163) (width 0.25) (layer B.Cu) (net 17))
 (segment (start 140.1318 105.0163) (end 140.1318 103.759) (width 0.25) (layer B.Cu) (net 17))
 (segment (start 140.1318 103.759) (end 138.483841 102.111041) (width 0.25) (layer B.Cu) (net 17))
 (segment (start 123.202611 102.111041) (end 138.483841 102.111041) (width 0.25) (layer B.Cu) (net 17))
 (segment (start 120.65 99.55843) (end 123.202611 102.111041) (width 0.25) (layer B.Cu) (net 17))
 (segment (start 120.65 97.358) (end 120.65 99.55843) (width 0.25) (layer B.Cu) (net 17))
 (segment (start 120.65 98.56732) (end 120.65 97.358) (width 0.2) (layer B.Cu) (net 17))
 (segment (start 119.255379 100.953051) (end 120.65 99.55843) (width 0.2) (layer B.Cu) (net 17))
 (segment (start 114.52332 100.953051) (end 119.255379 100.953051) (width 0.2) (layer B.Cu) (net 17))
 (segment (start 113.01843 99.448161) (end 114.52332 100.953051) (width 0.2) (layer B.Cu) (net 17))
 (segment (start 113.01843 97.73815) (end 113.01843 99.448161) (width 0.2) (layer B.Cu) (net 17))
 (segment (start 113.97566 96.78092) (end 113.01843 97.73815) (width 0.2) (layer B.Cu) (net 17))
 (segment (start 114.47566 96.78092) (end 113.97566 96.78092) (width 0.2) (layer B.Cu) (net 17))
 (via (at 127.4699 96.7867) (size 0.4) (drill 0.254) (layers F.Cu B.Cu) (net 6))
 (segment (start 127.4692 96.786) (end 127.4699 96.7867) (width 0.25) (layer F.Cu) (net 6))
 (segment (start 126.6202 96.786) (end 127.4692 96.786) (width 0.25) (layer F.Cu) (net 6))
 (segment (start 127.4699 96.7867) (end 127.4699 95.5929) (width 0.25) (layer B.Cu) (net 6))
 (segment (start 127.4699 95.5929) (end 127.03251 95.15551) (width 0.25) (layer B.Cu) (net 6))
 (segment (start 118.71249 95.15551) (end 117.983 95.885) (width 0.25) (layer B.Cu) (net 6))
 (segment (start 127.03251 95.15551) (end 118.71249 95.15551) (width 0.25) (layer B.Cu) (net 6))
 (segment (start 117.983 95.885) (end 117.983 96.805919) (width 0.25) (layer B.Cu) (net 6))
 (segment (start 117.83295 96.805919) (end 117.83295 96.745594) (width 0.25) (layer B.Cu) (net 6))
 (segment (start 117.983 96.805919) (end 117.83295 96.805919) (width 0.25) (layer B.Cu) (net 6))
 (segment (start 127.821199 97.311701) (end 127.8382 97.2947) (width 0.25) (layer F.Cu) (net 7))
 (segment (start 126.645901 97.311701) (end 127.821199 97.311701) (width 0.25) (layer F.Cu) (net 7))
 (via (at 127.8382 97.2947) (size 0.4) (drill 0.254) (layers F.Cu B.Cu) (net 7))
 (segment (start 126.6202 97.286) (end 126.645901 97.311701) (width 0.25) (layer F.Cu) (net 7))
 (segment (start 127.8382 97.2947) (end 127.821199 97.311701) (width 0.25) (layer B.Cu) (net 7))
 (segment (start 126.873 96.966802) (end 126.873 95.63241) (width 0.25) (layer B.Cu) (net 7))
 (segment (start 127.721901 97.311701) (end 127.217899 97.311701) (width 0.25) (layer B.Cu) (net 7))
 (segment (start 127.217899 97.311701) (end 126.873 96.966802) (width 0.25) (layer B.Cu) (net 7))
 (segment (start 127.738902 97.2947) (end 127.721901 97.311701) (width 0.25) (layer B.Cu) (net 7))
 (segment (start 127.8382 97.2947) (end 127.738902 97.2947) (width 0.25) (layer B.Cu) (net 7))
 (segment (start 126.873 95.63241) (end 126.84611 95.60552) (width 0.25) (layer B.Cu) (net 7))
 (segment (start 126.84611 95.60552) (end 118.89889 95.60552) (width 0.25) (layer B.Cu) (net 7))
 (segment (start 118.89889 95.60552) (end 118.43301 96.0714) (width 0.25) (layer B.Cu) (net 7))
 (segment (start 118.144409 97.28092) (end 117.83295 97.28092) (width 0.25) (layer B.Cu) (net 7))
 (segment (start 118.43301 96.992319) (end 118.144409 97.28092) (width 0.25) (layer B.Cu) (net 7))
 (segment (start 118.43301 96.0714) (end 118.43301 96.992319) (width 0.25) (layer B.Cu) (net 7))
 (via (at 128.1557 97.8154) (size 0.4) (drill 0.254) (layers F.Cu B.Cu) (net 8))
 (segment (start 128.151399 97.819701) (end 128.1557 97.8154) (width 0.25) (layer F.Cu) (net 8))
 (segment (start 126.653901 97.819701) (end 128.151399 97.819701) (width 0.25) (layer F.Cu) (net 8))
 (segment (start 126.6202 97.786) (end 126.653901 97.819701) (width 0.25) (layer F.Cu) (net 8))
 (segment (start 128.094502 97.8154) (end 128.090201 97.819701) (width 0.25) (layer B.Cu) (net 8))
 (segment (start 128.1557 97.8154) (end 128.094502 97.8154) (width 0.25) (layer B.Cu) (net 8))
 (segment (start 118.883019 97.17872) (end 118.271739 97.79) (width 0.25) (layer B.Cu) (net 8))
 (segment (start 121.58253 96.05553) (end 119.08529 96.05553) (width 0.25) (layer B.Cu) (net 8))
 (segment (start 121.59699 96.06999) (end 121.58253 96.05553) (width 0.25) (layer B.Cu) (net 8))
 (segment (start 126.42299 96.06999) (end 121.59699 96.06999) (width 0.25) (layer B.Cu) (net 8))
 (segment (start 126.42299 97.153202) (end 126.42299 96.06999) (width 0.25) (layer B.Cu) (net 8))
 (segment (start 119.08529 96.05553) (end 118.88302 96.2578) (width 0.25) (layer B.Cu) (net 8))
 (segment (start 127.089489 97.819701) (end 126.42299 97.153202) (width 0.25) (layer B.Cu) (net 8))
 (segment (start 118.88302 96.2578) (end 118.883019 97.17872) (width 0.25) (layer B.Cu) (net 8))
 (segment (start 128.151399 97.819701) (end 127.089489 97.819701) (width 0.25) (layer B.Cu) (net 8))
 (segment (start 118.271739 97.79) (end 117.83295 97.79) (width 0.25) (layer B.Cu) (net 8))
 (segment (start 128.1557 97.8154) (end 128.151399 97.819701) (width 0.25) (layer B.Cu) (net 8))
 (via (at 128.195611 98.414073) (size 0.4) (drill 0.254) (layers F.Cu B.Cu) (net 9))
 (segment (start 126.748273 98.414073) (end 128.195611 98.414073) (width 0.25) (layer F.Cu) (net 9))
 (segment (start 126.6202 98.286) (end 126.748273 98.414073) (width 0.25) (layer F.Cu) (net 9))
 (segment (start 117.83295 98.28092) (end 117.83295 98.326406) (width 0.25) (layer B.Cu) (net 9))
 (segment (start 118.417229 98.28092) (end 117.83295 98.28092) (width 0.25) (layer B.Cu) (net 9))
 (segment (start 119.333028 97.365121) (end 118.417229 98.28092) (width 0.25) (layer B.Cu) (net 9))
 (segment (start 119.333029 96.820971) (end 119.333028 97.365121) (width 0.25) (layer B.Cu) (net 9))
 (segment (start 119.64846 96.50554) (end 119.333029 96.820971) (width 0.25) (layer B.Cu) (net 9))
 (segment (start 120.38154 96.50554) (end 119.64846 96.50554) (width 0.25) (layer B.Cu) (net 9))
 (segment (start 120.396 96.52) (end 120.38154 96.50554) (width 0.25) (layer B.Cu) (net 9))
 (segment (start 125.857 96.52) (end 120.396 96.52) (width 0.25) (layer B.Cu) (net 9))
 (segment (start 125.97298 96.63598) (end 125.857 96.52) (width 0.25) (layer B.Cu) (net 9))
 (segment (start 125.97298 97.339602) (end 125.97298 96.63598) (width 0.25) (layer B.Cu) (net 9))
 (segment (start 127.047451 98.414073) (end 125.97298 97.339602) (width 0.25) (layer B.Cu) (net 9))
 (segment (start 128.195611 98.414073) (end 127.047451 98.414073) (width 0.25) (layer B.Cu) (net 9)))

